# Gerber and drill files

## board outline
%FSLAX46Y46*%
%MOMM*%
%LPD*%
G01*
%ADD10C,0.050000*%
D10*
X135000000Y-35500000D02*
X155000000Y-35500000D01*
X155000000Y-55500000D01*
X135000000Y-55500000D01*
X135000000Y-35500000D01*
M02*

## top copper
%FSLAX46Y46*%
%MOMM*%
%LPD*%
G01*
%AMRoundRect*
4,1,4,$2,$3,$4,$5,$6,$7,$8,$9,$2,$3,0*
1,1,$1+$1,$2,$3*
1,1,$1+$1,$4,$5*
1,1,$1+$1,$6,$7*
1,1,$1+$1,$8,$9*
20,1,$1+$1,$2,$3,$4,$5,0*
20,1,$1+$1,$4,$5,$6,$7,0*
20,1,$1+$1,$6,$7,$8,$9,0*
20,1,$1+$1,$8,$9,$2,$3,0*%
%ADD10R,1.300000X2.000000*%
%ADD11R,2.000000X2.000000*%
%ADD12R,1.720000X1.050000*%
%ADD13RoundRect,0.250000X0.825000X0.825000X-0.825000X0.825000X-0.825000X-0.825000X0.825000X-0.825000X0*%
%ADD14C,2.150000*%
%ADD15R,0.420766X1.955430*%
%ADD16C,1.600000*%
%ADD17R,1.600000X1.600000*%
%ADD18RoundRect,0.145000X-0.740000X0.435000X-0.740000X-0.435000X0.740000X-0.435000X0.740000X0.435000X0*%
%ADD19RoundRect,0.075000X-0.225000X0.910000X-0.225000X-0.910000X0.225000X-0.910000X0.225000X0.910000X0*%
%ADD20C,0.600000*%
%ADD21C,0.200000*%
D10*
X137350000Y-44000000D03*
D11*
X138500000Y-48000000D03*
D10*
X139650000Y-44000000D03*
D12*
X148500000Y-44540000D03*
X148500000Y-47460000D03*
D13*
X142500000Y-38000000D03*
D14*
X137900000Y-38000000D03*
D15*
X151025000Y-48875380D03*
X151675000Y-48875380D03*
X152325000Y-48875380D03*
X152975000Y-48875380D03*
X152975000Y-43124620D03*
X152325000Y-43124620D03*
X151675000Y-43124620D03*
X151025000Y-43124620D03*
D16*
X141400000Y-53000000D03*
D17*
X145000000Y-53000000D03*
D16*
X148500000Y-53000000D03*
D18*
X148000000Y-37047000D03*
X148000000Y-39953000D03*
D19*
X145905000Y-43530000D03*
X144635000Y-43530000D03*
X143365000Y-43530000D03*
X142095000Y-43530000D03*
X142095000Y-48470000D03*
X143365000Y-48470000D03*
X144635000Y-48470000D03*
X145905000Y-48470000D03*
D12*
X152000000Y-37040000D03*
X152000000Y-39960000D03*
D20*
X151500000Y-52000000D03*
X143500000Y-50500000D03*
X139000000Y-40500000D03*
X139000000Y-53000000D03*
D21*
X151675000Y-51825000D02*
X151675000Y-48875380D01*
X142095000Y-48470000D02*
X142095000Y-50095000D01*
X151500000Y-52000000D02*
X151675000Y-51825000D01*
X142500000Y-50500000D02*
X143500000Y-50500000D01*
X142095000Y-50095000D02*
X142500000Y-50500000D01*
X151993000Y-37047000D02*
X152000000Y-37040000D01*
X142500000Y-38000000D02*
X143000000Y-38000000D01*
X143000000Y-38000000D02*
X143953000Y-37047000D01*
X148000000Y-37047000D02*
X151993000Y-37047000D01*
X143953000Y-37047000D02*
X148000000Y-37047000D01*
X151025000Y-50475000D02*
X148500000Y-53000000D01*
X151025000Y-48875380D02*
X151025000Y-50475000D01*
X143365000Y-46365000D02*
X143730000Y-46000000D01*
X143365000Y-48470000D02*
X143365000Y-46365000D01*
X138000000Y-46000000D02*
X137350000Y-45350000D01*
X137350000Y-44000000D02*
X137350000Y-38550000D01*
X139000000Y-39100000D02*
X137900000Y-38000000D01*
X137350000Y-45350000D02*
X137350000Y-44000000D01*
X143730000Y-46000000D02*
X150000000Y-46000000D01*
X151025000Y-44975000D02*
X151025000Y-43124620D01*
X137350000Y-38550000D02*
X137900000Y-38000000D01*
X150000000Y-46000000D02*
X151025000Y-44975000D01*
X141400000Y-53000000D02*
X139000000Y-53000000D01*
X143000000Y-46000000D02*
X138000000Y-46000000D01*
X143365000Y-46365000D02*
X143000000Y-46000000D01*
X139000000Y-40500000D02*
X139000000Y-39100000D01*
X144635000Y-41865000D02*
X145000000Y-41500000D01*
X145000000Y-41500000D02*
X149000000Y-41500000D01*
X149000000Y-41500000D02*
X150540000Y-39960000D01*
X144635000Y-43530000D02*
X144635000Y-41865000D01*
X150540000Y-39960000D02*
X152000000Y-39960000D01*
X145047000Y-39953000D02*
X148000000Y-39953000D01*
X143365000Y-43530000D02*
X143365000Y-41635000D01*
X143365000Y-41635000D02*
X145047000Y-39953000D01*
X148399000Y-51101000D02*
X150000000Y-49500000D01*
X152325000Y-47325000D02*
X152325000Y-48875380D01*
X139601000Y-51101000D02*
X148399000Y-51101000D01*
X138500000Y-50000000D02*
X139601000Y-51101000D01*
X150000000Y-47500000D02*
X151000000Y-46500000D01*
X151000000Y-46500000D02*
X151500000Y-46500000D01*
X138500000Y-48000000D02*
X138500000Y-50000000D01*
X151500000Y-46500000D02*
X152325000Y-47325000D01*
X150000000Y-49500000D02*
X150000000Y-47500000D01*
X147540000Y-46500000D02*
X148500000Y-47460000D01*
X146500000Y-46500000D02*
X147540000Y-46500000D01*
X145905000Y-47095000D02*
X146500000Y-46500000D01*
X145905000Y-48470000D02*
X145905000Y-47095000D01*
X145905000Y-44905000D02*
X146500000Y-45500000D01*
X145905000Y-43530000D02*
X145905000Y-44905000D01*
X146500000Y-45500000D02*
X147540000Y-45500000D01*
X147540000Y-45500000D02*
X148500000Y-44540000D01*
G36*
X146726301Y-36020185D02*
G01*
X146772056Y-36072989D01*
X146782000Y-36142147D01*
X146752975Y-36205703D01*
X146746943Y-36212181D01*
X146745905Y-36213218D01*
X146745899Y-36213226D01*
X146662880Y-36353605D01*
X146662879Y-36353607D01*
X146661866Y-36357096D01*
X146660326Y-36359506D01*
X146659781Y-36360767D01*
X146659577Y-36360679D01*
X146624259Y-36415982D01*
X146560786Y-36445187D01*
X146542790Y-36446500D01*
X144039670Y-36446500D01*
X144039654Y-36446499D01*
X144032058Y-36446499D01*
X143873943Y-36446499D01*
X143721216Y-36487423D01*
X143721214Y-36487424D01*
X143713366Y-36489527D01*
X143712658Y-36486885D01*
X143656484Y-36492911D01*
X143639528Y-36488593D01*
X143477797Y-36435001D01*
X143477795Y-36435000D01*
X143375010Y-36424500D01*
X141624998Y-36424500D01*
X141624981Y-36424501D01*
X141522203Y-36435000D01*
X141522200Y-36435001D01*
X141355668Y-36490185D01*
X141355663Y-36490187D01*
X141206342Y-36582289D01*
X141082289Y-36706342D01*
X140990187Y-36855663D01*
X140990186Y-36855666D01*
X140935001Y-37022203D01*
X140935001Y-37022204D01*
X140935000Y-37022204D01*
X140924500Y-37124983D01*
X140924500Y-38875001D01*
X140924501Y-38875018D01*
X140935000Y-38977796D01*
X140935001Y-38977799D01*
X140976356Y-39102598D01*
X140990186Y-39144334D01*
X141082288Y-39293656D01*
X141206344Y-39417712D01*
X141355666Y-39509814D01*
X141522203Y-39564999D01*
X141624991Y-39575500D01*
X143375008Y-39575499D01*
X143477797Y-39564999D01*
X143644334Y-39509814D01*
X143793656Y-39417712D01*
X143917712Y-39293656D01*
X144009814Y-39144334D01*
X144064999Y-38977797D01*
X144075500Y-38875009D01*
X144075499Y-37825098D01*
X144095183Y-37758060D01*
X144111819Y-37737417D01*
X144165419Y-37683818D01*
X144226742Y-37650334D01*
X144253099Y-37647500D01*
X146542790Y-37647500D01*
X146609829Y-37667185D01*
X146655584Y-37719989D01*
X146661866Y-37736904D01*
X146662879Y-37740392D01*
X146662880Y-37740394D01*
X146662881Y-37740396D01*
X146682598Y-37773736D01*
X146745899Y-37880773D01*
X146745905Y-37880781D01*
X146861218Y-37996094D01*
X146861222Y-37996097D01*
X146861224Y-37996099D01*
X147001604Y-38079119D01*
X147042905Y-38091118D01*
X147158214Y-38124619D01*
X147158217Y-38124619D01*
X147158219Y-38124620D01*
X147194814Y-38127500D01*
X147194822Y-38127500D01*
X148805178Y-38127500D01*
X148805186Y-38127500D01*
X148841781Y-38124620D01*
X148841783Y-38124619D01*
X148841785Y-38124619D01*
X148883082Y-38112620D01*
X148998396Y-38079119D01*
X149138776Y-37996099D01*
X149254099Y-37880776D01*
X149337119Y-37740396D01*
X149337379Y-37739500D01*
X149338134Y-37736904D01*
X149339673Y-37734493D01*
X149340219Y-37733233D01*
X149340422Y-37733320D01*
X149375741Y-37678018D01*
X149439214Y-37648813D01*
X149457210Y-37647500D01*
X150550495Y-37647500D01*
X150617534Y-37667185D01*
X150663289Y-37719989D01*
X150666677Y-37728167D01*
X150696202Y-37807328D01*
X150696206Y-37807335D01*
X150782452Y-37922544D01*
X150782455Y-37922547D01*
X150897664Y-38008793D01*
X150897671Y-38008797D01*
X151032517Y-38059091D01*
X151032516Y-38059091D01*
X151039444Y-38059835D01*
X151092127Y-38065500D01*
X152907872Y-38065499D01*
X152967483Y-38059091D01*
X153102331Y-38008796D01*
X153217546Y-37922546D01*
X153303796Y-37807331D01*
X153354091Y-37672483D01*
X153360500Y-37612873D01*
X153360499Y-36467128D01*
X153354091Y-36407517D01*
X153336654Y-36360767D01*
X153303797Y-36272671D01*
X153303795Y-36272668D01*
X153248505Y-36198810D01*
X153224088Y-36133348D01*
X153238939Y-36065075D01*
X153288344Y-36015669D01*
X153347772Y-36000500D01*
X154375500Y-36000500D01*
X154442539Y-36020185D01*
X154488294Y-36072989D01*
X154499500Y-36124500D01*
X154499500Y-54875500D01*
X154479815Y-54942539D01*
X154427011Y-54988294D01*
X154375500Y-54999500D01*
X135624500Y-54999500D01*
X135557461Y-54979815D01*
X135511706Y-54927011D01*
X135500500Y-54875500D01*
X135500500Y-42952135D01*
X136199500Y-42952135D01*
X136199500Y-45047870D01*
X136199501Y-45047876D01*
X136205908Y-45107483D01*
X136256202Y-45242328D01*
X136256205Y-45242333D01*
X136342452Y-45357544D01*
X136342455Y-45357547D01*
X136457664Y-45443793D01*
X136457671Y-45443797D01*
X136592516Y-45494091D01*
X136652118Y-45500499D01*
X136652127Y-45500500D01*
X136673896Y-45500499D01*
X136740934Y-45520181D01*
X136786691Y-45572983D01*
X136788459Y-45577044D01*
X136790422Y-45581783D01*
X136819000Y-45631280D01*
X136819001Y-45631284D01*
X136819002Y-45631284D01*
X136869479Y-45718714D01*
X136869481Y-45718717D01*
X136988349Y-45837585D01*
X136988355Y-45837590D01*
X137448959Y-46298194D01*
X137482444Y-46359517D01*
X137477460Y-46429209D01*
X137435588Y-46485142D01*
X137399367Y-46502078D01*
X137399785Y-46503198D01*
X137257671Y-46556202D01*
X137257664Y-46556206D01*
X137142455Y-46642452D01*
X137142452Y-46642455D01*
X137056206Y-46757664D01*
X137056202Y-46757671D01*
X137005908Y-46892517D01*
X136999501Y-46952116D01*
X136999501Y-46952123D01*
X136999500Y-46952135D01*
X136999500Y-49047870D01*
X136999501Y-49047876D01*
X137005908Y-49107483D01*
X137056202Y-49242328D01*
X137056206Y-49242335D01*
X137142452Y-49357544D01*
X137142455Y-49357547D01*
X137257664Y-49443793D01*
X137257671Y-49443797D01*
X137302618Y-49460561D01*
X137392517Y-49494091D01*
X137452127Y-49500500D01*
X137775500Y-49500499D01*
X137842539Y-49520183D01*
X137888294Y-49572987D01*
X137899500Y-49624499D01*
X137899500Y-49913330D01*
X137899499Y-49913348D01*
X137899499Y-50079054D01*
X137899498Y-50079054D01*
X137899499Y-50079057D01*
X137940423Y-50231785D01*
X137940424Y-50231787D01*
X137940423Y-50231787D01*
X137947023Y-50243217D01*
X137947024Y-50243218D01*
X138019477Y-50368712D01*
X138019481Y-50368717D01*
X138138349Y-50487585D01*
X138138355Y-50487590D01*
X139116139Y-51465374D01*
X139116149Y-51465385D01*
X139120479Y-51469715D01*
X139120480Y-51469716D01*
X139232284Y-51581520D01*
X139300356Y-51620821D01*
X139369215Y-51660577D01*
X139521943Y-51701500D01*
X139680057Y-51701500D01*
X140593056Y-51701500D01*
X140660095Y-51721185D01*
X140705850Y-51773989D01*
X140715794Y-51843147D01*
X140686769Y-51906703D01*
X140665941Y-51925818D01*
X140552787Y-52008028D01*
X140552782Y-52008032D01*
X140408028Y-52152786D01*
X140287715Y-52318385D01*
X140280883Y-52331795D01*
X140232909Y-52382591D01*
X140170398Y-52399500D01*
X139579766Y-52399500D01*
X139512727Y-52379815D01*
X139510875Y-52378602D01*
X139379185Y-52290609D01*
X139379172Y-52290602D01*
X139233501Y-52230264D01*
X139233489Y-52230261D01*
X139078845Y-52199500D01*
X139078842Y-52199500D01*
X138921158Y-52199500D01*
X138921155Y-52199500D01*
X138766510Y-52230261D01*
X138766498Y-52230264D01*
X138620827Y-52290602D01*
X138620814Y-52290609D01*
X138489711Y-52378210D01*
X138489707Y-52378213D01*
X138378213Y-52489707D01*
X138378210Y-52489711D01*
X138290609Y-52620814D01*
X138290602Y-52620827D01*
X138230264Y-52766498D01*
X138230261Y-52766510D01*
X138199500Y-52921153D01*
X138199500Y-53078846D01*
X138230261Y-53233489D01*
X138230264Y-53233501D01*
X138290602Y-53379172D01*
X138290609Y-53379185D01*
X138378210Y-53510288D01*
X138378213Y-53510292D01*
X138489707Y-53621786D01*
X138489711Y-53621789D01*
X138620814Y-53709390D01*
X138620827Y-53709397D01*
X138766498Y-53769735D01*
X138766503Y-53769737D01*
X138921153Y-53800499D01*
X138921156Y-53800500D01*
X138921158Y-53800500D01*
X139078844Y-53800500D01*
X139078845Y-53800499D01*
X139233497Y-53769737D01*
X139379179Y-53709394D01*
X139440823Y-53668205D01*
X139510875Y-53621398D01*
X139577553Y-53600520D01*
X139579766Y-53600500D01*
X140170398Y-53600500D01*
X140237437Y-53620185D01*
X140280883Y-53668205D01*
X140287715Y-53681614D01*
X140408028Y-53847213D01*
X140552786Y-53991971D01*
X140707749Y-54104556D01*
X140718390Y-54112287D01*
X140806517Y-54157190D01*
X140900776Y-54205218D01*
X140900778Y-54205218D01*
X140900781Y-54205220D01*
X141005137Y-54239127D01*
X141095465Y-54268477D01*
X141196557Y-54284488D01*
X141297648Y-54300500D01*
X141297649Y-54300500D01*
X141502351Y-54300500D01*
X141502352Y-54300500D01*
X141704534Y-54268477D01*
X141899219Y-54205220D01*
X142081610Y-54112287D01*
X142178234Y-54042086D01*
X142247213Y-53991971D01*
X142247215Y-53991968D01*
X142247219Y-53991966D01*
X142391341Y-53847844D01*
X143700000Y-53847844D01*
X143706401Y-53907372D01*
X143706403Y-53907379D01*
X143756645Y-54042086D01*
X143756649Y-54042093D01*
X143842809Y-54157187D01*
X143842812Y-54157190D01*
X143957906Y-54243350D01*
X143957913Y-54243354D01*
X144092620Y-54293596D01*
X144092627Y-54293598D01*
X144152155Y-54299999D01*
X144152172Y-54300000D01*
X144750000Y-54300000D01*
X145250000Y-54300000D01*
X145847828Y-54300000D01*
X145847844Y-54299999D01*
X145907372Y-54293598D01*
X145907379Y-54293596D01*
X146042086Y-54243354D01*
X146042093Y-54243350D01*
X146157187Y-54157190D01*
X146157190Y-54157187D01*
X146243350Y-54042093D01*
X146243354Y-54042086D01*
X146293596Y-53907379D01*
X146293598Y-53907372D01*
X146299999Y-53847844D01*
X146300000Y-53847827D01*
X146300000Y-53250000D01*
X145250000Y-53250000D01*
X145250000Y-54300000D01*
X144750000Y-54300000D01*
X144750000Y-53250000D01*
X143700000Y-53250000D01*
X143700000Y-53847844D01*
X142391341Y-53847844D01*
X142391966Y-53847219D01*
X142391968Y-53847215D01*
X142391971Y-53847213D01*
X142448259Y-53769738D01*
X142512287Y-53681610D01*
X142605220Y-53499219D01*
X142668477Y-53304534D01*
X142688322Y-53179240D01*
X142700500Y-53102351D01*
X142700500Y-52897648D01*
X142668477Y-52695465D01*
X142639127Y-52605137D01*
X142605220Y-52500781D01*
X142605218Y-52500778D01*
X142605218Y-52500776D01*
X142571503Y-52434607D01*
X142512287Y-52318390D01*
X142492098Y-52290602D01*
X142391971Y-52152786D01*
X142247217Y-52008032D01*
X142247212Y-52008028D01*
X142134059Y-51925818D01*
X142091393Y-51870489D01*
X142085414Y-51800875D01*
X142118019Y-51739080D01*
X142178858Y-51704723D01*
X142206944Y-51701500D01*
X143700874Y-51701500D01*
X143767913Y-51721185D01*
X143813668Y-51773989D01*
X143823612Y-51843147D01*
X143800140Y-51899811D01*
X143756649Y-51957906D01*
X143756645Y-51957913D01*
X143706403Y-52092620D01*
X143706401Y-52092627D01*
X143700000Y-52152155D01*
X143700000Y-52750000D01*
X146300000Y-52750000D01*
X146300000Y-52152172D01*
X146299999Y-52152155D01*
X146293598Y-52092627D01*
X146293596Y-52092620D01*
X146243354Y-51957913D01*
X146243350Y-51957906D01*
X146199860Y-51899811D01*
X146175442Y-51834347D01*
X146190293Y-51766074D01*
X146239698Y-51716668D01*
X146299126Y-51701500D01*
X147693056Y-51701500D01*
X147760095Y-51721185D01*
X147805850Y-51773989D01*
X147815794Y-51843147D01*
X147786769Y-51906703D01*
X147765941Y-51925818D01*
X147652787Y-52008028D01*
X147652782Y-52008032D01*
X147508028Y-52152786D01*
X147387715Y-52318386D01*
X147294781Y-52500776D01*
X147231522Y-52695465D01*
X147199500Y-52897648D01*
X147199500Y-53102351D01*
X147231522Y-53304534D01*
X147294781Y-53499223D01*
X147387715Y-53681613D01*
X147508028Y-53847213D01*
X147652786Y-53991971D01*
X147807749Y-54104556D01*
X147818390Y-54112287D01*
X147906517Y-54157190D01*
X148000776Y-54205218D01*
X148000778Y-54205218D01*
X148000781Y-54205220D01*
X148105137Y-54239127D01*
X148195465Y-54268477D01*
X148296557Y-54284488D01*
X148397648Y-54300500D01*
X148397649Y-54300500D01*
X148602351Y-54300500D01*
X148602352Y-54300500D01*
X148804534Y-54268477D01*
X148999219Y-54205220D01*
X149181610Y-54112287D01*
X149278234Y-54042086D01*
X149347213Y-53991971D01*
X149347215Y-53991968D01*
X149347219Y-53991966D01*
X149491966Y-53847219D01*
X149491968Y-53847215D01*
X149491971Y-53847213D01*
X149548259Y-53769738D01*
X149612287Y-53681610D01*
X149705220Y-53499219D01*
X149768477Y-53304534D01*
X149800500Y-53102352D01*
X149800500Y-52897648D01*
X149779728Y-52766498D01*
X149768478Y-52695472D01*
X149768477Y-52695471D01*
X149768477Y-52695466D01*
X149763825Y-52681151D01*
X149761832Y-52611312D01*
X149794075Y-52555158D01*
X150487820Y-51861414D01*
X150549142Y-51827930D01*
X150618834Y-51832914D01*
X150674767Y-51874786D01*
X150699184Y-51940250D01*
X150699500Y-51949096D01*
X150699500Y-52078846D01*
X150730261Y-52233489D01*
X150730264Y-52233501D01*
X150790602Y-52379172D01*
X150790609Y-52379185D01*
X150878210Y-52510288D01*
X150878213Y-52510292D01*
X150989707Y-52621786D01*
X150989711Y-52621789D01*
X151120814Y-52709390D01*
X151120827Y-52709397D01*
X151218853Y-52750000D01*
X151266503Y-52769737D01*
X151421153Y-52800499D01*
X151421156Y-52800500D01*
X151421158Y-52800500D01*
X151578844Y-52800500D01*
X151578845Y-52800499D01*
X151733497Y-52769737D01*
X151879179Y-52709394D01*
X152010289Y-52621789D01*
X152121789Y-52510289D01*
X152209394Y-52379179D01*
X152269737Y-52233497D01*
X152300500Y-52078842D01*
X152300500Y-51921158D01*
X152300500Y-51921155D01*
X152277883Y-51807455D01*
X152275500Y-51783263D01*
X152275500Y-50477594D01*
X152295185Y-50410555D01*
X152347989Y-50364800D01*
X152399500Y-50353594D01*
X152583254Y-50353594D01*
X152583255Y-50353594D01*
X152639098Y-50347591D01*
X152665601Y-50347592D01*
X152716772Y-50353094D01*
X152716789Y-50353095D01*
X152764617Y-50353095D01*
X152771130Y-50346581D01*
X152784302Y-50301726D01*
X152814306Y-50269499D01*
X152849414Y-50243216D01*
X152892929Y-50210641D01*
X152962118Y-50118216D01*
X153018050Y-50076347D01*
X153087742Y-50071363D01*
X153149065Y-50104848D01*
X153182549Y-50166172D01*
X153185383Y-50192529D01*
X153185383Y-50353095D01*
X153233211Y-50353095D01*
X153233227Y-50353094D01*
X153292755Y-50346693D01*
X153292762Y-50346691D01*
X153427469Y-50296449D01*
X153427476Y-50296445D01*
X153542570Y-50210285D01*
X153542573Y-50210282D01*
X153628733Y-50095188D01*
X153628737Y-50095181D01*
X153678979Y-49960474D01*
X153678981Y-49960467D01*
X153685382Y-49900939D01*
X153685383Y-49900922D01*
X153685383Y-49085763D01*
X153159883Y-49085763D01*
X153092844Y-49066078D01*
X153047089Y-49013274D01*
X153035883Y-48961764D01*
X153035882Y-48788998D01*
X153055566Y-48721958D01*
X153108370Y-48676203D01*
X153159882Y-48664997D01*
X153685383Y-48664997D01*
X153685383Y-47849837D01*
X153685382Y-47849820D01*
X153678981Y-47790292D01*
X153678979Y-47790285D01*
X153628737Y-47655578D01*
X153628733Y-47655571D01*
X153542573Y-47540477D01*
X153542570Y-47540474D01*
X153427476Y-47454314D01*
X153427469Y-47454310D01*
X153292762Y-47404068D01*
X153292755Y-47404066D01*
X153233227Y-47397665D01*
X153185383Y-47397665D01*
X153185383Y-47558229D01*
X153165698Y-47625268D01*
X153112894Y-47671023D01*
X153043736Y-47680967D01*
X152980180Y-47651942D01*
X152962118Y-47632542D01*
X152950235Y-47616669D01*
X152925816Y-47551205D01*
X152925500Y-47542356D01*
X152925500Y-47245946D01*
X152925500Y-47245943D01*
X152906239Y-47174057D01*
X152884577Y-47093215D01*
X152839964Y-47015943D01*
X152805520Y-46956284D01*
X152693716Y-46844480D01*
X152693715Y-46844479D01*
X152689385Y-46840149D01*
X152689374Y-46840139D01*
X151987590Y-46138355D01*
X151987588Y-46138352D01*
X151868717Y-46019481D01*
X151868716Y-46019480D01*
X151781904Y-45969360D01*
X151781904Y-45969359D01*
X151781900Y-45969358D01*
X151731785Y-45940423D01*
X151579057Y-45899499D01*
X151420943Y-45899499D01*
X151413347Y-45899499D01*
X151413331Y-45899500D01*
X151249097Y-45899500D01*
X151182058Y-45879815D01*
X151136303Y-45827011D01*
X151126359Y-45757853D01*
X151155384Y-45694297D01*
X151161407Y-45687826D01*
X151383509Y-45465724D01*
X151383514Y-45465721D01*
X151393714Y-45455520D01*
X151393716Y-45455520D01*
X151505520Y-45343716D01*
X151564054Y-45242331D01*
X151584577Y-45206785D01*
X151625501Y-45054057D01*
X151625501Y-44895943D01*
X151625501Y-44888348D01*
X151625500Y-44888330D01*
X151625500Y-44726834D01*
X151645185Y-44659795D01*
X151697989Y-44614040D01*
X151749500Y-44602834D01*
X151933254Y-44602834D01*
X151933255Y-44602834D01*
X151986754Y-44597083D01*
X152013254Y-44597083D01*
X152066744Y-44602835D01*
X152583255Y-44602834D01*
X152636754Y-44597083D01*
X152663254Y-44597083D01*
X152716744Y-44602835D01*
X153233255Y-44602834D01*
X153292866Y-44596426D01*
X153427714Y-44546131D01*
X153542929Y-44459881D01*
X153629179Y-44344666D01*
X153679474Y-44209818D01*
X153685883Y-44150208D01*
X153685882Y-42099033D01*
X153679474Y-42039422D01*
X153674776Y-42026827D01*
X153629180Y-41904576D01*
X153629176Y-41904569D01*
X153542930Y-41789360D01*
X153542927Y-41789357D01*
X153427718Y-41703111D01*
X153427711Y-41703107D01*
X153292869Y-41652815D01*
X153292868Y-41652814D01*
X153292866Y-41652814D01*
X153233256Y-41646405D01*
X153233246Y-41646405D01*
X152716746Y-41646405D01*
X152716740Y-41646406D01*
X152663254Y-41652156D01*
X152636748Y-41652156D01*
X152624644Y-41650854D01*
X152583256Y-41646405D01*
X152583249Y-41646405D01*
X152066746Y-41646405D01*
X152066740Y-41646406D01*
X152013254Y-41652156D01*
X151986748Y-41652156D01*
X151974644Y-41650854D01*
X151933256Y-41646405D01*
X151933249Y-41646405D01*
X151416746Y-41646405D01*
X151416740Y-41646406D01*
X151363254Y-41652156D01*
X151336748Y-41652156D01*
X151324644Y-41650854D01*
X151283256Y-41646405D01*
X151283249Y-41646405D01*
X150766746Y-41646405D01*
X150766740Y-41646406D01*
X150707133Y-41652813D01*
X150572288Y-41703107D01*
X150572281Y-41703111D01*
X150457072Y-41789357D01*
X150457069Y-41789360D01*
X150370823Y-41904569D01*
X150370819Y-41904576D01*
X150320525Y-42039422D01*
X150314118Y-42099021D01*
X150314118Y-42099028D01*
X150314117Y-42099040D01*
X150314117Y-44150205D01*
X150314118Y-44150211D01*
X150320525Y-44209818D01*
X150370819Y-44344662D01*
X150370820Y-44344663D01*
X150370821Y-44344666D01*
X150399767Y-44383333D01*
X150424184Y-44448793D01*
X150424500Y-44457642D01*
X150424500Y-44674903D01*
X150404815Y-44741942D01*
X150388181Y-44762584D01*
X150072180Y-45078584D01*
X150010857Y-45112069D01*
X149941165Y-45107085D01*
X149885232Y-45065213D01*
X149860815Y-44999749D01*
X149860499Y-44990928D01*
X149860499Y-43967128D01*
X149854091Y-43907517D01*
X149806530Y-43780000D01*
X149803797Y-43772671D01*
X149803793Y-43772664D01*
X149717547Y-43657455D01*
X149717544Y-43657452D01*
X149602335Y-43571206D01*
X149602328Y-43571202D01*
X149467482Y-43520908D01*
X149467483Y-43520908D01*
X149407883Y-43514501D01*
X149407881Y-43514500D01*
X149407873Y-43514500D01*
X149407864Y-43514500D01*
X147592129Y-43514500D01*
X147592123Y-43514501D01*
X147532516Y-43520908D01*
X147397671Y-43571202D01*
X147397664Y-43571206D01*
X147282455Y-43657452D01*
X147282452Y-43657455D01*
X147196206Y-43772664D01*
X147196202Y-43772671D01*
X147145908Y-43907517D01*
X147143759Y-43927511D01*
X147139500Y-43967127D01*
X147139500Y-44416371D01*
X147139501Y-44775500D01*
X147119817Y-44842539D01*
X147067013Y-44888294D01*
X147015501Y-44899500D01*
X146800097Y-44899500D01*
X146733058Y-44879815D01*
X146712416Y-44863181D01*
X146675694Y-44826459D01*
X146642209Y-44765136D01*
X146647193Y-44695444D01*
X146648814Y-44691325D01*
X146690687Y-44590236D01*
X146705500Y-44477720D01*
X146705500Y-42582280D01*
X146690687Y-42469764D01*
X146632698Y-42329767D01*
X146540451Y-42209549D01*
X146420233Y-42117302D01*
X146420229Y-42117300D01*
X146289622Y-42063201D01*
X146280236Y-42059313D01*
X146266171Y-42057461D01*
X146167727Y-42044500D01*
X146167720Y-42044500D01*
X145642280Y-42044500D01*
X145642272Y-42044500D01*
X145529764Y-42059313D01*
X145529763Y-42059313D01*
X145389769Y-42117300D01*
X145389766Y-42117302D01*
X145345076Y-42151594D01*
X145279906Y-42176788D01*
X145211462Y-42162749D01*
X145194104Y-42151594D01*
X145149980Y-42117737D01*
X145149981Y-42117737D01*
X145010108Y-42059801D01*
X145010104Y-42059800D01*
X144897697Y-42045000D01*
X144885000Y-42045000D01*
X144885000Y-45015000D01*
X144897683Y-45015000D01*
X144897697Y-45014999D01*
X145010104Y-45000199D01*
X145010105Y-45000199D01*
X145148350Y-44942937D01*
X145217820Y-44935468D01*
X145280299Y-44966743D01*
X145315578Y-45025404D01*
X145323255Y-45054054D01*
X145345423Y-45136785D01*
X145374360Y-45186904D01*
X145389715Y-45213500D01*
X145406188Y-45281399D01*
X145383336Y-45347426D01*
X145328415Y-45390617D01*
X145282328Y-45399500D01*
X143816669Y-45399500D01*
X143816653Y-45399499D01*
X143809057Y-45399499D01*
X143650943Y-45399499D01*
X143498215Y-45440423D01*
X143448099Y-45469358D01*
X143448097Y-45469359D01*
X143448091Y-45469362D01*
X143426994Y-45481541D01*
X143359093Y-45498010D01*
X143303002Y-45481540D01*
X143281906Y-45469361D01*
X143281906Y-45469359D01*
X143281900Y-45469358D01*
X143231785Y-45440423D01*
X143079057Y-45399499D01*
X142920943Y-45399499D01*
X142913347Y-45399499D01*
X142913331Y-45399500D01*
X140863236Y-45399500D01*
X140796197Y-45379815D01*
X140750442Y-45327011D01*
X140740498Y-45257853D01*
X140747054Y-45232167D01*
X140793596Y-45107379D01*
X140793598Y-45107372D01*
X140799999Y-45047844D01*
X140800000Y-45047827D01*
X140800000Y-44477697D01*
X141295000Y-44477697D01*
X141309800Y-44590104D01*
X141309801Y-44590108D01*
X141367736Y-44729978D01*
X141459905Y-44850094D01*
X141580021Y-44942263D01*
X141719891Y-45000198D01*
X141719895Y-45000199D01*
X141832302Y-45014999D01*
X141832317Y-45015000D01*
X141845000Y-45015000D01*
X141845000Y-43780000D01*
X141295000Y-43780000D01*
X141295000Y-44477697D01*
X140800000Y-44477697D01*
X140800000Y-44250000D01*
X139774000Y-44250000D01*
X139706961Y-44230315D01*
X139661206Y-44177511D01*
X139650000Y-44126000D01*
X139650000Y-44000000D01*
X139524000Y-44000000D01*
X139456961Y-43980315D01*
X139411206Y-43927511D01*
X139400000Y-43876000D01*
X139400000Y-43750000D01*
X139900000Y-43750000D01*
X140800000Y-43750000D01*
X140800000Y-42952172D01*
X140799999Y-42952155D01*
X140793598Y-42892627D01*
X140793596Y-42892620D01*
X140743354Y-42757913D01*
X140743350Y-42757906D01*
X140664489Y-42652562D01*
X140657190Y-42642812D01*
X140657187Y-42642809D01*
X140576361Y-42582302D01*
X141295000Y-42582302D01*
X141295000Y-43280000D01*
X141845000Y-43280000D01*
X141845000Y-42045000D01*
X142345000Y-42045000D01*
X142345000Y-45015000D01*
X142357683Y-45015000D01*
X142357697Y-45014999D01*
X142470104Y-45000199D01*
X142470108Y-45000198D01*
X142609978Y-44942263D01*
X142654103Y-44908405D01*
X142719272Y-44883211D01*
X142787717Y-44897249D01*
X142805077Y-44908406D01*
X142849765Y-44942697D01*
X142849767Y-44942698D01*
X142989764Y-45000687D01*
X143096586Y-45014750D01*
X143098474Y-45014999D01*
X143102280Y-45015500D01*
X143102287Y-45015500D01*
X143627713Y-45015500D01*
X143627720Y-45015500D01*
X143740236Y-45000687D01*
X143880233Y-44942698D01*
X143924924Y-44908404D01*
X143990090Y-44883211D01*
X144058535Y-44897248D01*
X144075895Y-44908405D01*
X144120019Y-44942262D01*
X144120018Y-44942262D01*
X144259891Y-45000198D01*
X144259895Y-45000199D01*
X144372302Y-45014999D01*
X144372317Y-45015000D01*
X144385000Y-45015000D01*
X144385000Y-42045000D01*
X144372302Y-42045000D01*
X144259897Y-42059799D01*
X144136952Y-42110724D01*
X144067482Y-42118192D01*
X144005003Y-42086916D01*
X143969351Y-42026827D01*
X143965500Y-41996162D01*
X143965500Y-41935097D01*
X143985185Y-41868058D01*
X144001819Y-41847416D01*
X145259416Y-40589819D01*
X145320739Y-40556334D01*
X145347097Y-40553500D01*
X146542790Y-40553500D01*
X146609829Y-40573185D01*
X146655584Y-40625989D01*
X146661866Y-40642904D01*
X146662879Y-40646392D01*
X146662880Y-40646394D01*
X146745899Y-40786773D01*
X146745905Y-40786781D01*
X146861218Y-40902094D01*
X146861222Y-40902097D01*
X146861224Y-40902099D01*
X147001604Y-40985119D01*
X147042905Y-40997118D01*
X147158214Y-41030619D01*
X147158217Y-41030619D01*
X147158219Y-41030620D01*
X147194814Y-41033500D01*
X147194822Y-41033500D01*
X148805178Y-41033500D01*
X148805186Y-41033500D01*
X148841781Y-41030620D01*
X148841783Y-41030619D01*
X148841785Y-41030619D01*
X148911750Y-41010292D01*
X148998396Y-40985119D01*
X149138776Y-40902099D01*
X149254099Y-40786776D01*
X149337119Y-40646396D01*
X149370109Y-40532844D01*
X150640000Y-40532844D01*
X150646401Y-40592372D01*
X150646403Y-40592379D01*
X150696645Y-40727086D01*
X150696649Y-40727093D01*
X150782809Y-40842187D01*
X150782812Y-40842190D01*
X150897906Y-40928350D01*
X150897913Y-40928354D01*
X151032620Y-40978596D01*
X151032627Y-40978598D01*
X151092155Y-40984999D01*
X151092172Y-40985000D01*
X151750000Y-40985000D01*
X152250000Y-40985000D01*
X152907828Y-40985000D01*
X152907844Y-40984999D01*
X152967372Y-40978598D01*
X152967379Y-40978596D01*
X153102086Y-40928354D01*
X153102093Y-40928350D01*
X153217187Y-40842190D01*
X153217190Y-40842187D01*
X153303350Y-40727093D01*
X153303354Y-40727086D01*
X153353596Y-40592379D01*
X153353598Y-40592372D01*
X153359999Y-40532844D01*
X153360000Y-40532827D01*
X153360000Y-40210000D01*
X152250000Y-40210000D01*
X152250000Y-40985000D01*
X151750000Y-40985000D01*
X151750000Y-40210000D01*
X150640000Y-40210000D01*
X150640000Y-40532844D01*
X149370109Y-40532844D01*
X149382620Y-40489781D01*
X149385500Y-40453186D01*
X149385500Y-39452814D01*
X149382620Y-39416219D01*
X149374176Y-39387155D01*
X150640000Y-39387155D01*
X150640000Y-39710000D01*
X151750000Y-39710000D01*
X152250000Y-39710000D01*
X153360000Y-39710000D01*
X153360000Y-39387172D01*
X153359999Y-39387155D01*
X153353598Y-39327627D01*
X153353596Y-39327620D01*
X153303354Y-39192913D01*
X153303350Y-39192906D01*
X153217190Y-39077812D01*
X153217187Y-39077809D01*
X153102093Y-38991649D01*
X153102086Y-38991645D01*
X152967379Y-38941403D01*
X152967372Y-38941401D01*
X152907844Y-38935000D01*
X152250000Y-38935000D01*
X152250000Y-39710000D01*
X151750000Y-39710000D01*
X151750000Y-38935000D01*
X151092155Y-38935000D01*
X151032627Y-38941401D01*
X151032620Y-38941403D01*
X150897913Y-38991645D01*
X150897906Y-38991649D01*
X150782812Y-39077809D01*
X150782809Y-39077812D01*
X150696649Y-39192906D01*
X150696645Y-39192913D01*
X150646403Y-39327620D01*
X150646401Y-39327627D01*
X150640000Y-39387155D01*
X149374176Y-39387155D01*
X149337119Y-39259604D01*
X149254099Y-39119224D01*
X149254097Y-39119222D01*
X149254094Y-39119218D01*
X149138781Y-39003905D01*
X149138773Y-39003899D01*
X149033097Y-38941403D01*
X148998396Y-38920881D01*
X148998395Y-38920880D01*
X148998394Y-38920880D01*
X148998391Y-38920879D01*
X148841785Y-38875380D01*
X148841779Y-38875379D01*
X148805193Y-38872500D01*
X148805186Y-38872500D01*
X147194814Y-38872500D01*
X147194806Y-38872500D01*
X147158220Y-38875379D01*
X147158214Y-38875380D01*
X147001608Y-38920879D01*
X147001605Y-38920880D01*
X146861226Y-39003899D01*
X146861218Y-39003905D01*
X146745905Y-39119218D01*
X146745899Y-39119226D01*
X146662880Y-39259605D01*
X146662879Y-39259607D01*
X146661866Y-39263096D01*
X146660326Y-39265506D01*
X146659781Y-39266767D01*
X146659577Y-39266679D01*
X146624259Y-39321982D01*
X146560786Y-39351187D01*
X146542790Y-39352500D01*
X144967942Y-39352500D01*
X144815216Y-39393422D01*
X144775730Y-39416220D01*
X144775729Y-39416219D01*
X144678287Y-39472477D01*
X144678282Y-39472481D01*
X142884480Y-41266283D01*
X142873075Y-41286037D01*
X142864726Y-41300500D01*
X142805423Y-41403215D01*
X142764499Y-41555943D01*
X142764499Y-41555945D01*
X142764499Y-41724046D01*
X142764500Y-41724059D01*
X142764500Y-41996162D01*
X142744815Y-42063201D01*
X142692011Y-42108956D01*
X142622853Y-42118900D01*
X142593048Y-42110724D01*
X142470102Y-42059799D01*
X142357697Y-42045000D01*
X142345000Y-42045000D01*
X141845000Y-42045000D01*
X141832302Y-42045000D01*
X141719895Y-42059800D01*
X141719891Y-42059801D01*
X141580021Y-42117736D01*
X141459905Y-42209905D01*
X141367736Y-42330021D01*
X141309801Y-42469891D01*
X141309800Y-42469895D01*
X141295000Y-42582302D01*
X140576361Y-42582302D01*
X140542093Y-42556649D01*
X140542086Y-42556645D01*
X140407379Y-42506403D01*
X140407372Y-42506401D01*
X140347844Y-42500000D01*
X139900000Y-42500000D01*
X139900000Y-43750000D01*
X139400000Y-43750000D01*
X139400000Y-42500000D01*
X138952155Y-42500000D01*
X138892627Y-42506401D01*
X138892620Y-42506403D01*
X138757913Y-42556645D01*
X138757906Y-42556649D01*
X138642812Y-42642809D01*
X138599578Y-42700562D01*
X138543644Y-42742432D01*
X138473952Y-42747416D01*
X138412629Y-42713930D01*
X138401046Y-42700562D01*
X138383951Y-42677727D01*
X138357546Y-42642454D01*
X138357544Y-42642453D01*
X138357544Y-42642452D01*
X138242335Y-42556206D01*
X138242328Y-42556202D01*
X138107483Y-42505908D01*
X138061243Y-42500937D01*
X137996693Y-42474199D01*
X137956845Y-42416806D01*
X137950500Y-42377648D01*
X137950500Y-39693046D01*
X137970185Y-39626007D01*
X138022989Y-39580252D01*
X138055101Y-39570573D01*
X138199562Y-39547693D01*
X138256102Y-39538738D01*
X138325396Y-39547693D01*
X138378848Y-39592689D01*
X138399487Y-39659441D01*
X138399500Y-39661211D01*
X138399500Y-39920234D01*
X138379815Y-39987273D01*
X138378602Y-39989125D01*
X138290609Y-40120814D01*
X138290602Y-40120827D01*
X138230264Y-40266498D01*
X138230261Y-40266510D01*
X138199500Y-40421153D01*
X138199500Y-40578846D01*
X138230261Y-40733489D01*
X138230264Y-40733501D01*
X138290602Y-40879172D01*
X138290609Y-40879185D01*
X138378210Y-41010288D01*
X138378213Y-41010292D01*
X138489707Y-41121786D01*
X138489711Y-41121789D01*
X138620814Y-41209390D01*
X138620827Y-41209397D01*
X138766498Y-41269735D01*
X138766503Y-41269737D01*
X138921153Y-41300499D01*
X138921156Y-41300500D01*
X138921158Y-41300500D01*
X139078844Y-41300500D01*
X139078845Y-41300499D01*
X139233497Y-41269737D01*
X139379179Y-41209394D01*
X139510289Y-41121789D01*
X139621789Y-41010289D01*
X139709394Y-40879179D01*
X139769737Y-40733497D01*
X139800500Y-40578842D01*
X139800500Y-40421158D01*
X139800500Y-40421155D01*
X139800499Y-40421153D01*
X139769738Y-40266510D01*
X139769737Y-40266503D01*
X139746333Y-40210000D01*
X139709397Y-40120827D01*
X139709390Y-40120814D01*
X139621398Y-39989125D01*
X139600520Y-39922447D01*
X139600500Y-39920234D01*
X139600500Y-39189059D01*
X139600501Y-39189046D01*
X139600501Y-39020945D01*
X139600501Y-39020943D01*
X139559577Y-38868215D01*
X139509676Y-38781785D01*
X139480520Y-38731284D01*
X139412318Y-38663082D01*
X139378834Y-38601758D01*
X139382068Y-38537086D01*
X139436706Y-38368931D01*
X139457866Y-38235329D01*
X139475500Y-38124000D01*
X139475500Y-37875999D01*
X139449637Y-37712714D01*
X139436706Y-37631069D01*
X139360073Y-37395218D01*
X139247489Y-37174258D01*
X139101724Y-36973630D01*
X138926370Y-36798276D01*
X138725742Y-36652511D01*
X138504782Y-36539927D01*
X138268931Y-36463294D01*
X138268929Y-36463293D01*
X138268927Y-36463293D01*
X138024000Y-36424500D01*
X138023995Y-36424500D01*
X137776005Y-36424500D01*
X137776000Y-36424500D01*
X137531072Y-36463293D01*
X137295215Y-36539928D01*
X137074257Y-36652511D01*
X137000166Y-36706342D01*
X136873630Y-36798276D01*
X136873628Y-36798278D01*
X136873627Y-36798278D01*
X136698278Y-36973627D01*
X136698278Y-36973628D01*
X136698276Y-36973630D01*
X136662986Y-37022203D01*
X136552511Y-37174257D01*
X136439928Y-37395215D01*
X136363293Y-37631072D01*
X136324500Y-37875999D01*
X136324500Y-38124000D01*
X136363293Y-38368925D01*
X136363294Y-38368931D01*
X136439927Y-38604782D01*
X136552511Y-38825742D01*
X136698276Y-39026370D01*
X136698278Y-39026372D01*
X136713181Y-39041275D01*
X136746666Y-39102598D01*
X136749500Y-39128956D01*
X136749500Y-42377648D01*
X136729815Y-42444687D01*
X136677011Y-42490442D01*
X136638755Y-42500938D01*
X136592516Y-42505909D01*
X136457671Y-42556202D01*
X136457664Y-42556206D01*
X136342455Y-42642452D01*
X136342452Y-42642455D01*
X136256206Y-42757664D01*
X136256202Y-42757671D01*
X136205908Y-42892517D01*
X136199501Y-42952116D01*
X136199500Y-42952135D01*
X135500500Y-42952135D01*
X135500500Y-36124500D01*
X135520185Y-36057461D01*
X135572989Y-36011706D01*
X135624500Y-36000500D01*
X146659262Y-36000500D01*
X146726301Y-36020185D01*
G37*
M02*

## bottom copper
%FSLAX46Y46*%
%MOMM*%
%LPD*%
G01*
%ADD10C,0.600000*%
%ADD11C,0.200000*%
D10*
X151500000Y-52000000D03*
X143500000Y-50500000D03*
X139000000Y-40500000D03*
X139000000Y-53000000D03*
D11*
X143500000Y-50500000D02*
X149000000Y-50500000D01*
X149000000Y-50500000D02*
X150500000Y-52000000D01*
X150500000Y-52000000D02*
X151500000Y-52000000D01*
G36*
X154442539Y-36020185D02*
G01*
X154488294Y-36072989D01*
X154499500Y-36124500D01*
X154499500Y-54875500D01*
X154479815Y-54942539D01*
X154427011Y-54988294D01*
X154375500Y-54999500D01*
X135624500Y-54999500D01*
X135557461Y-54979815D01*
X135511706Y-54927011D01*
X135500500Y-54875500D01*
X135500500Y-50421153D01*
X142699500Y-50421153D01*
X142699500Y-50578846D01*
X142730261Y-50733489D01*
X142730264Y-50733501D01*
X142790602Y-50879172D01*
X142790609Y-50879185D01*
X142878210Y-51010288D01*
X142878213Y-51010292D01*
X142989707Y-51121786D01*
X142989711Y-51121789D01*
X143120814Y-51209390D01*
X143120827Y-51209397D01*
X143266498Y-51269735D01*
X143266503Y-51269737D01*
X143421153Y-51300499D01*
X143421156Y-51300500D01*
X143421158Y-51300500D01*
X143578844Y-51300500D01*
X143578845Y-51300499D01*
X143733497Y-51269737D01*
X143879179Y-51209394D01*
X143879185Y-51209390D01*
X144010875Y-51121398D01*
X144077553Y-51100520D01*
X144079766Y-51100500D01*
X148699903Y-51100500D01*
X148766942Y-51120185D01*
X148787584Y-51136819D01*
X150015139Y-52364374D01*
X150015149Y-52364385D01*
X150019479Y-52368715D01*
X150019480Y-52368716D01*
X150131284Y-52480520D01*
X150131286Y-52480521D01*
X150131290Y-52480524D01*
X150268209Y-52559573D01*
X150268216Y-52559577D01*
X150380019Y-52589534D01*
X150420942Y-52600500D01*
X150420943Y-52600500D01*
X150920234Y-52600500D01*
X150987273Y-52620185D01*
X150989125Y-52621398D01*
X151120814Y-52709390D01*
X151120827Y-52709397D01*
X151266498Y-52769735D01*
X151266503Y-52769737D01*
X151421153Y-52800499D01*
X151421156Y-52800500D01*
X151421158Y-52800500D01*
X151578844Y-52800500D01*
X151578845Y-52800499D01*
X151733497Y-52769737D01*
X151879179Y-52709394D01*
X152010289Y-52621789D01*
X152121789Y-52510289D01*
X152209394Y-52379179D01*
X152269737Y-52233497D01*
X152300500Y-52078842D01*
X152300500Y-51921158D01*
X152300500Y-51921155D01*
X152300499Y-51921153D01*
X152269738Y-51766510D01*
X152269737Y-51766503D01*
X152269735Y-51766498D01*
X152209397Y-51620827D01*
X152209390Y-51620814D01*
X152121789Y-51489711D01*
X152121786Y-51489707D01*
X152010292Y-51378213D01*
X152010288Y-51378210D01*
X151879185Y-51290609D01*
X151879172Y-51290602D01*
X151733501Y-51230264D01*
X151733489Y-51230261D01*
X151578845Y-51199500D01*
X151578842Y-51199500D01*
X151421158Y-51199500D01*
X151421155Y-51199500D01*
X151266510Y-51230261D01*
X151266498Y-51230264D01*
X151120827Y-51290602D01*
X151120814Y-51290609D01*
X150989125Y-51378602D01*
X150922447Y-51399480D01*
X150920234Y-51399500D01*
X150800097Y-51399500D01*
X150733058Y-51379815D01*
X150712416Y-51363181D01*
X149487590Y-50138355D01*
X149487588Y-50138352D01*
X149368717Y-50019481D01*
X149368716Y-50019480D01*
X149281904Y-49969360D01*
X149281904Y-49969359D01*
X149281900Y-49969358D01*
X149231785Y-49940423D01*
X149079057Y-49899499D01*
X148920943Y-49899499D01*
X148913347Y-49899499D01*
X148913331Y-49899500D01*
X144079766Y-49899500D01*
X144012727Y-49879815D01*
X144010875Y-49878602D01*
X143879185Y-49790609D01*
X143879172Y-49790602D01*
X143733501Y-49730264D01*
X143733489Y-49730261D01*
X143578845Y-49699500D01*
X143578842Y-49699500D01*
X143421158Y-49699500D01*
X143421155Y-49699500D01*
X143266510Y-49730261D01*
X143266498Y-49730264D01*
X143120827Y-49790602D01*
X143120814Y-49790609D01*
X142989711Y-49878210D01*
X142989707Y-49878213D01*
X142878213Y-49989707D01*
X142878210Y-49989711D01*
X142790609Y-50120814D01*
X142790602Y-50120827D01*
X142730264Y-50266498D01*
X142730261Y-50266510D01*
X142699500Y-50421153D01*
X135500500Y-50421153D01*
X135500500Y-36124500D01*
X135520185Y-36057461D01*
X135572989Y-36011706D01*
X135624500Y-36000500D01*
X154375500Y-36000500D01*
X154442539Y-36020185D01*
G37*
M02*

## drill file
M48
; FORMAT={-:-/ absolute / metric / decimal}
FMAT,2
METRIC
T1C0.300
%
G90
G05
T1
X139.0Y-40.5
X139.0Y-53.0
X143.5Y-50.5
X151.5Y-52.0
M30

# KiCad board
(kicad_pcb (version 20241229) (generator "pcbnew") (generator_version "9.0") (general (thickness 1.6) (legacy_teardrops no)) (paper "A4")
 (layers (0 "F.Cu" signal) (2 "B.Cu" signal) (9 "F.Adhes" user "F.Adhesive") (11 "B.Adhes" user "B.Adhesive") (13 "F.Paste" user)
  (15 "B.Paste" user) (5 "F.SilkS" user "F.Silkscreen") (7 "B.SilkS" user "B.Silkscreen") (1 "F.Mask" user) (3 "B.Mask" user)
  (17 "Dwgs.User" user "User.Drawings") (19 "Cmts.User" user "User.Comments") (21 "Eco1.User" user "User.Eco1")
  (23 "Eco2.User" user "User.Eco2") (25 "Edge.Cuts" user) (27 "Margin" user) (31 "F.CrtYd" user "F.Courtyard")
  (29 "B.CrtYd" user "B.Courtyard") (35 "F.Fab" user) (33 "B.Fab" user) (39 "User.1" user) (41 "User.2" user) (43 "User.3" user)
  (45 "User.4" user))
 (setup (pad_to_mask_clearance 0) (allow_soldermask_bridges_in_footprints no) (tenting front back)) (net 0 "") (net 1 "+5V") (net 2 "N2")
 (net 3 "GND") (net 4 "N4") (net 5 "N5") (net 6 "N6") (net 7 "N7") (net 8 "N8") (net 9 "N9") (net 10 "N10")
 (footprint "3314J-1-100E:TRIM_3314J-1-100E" (layer "F.Cu") (at 138.5 46 180)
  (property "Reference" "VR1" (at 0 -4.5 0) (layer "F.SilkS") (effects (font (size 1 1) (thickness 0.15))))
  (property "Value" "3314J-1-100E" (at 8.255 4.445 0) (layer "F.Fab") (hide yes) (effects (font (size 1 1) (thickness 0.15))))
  (pad "1" smd rect (at 1.15 2 180) (size 1.3 2) (layers "F.Cu" "F.Mask" "F.Paste") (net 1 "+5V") (solder_mask_margin 0.102))
  (pad "2" smd rect (at 0 -2 180) (size 2 2) (layers "F.Cu" "F.Mask" "F.Paste") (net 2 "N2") (solder_mask_margin 0.102))
  (pad "3" smd rect (at -1.15 2 180) (size 1.3 2) (layers "F.Cu" "F.Mask" "F.Paste") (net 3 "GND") (solder_mask_margin 0.102)))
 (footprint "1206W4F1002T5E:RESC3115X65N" (layer "F.Cu") (at 148.5 46 -90)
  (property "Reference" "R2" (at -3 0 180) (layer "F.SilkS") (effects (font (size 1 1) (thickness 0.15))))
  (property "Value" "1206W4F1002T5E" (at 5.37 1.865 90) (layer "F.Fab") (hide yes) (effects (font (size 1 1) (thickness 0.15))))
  (pad "1" smd rect (at -1.46 0 270) (size 1.05 1.72) (layers "F.Cu" "F.Mask" "F.Paste") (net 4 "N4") (solder_mask_margin 0.102))
  (pad "2" smd rect (at 1.46 0 270) (size 1.05 1.72) (layers "F.Cu" "F.Mask" "F.Paste") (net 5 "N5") (solder_mask_margin 0.102)))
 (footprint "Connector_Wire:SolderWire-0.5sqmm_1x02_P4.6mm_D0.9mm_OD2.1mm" (layer "F.Cu") (at 142.5 38 180)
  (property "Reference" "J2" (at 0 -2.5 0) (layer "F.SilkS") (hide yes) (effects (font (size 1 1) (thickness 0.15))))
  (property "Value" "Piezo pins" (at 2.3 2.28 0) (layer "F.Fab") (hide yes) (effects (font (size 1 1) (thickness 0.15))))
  (pad "1" smd roundrect (at 0 0 180) (size 2.15 2.15) (layers "F.Cu" "F.Mask" "F.Paste") (roundrect_rratio 0.116279) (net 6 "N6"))
  (pad "2" smd circle (at 4.6 0 180) (size 2.15 2.15) (layers "F.Cu" "F.Mask" "F.Paste") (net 1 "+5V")))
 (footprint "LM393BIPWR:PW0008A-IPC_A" (layer "F.Cu") (at 152 46 90)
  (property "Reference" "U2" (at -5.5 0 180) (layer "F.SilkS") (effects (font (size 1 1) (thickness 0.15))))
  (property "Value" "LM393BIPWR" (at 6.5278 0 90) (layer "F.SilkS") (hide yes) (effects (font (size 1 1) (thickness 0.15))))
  (pad "1" smd rect (at -2.87538 -0.975 90) (size 1.95543 0.420766) (layers "F.Cu" "F.Mask" "F.Paste") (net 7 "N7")
   (solder_mask_margin 0.102))
  (pad "2" smd rect (at -2.87538 -0.325 90) (size 1.95543 0.420766) (layers "F.Cu" "F.Mask" "F.Paste") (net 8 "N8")
   (solder_mask_margin 0.102))
  (pad "3" smd rect (at -2.87538 0.325 90) (size 1.95543 0.420766) (layers "F.Cu" "F.Mask" "F.Paste") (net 2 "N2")
   (solder_mask_margin 0.102))
  (pad "4" smd rect (at -2.87538 0.975 90) (size 1.95543 0.420766) (layers "F.Cu" "F.Mask" "F.Paste") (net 3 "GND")
   (solder_mask_margin 0.102))
  (pad "5" smd rect (at 2.87538 0.975 90) (size 1.95543 0.420766) (layers "F.Cu" "F.Mask" "F.Paste") (solder_mask_margin 0.102))
  (pad "6" smd rect (at 2.87538 0.325 90) (size 1.95543 0.420766) (layers "F.Cu" "F.Mask" "F.Paste") (solder_mask_margin 0.102))
  (pad "7" smd rect (at 2.87538 -0.325 90) (size 1.95543 0.420766) (layers "F.Cu" "F.Mask" "F.Paste") (solder_mask_margin 0.102))
  (pad "8" smd rect (at 2.87538 -0.975 90) (size 1.95543 0.420766) (layers "F.Cu" "F.Mask" "F.Paste") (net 1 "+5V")
   (solder_mask_margin 0.102)))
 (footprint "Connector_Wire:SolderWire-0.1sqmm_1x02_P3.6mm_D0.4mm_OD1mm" (layer "F.Cu") (at 141.4 53)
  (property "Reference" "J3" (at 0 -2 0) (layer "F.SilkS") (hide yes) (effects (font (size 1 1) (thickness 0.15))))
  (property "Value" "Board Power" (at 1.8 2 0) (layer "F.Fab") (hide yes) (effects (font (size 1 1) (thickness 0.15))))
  (pad "1" smd circle (at 0 0) (size 1.6 1.6) (layers "F.Cu" "F.Mask" "F.Paste") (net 1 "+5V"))
  (pad "2" smd rect (at 3.6 0) (size 1.6 1.6) (layers "F.Cu" "F.Mask" "F.Paste") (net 3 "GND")))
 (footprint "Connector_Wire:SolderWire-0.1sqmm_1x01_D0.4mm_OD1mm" (layer "F.Cu") (at 148.5 53)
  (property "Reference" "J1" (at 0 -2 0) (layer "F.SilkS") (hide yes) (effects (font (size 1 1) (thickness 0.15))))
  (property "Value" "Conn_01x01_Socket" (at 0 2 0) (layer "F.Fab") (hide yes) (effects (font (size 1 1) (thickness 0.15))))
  (pad "1" smd circle (at 0 0) (size 1.6 1.6) (layers "F.Cu" "F.Mask" "F.Paste") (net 7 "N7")))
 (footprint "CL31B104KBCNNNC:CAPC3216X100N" (layer "F.Cu") (at 148 38.5 -90)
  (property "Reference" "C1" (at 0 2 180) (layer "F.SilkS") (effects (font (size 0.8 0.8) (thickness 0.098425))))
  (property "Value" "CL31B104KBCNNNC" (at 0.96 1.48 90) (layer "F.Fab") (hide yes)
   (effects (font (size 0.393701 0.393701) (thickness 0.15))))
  (pad "1" smd roundrect (at -1.453 0 270) (size 1.16 1.77) (layers "F.Cu" "F.Mask" "F.Paste") (roundrect_rratio 0.125) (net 6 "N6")
   (solder_mask_margin 0.102))
  (pad "2" smd roundrect (at 1.453 0 270) (size 1.16 1.77) (layers "F.Cu" "F.Mask" "F.Paste") (roundrect_rratio 0.125) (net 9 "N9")
   (solder_mask_margin 0.102)))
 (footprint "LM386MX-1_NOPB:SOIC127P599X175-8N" (layer "F.Cu") (at 144 46 -90)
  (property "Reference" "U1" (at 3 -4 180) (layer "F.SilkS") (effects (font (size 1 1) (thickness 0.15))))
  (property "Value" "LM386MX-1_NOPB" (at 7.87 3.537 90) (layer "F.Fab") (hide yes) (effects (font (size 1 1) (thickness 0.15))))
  (pad "1" smd roundrect (at -2.47 -1.905 270) (size 1.97 0.6) (layers "F.Cu" "F.Mask" "F.Paste") (roundrect_rratio 0.125) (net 4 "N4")
   (solder_mask_margin 0.102))
  (pad "2" smd roundrect (at -2.47 -0.635 270) (size 1.97 0.6) (layers "F.Cu" "F.Mask" "F.Paste") (roundrect_rratio 0.125) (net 3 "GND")
   (solder_mask_margin 0.102))
  (pad "3" smd roundrect (at -2.47 0.635 270) (size 1.97 0.6) (layers "F.Cu" "F.Mask" "F.Paste") (roundrect_rratio 0.125) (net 9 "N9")
   (solder_mask_margin 0.102))
  (pad "4" smd roundrect (at -2.47 1.905 270) (size 1.97 0.6) (layers "F.Cu" "F.Mask" "F.Paste") (roundrect_rratio 0.125) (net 3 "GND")
   (solder_mask_margin 0.102))
  (pad "5" smd roundrect (at 2.47 1.905 270) (size 1.97 0.6) (layers "F.Cu" "F.Mask" "F.Paste") (roundrect_rratio 0.125) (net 8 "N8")
   (solder_mask_margin 0.102))
  (pad "6" smd roundrect (at 2.47 0.635 270) (size 1.97 0.6) (layers "F.Cu" "F.Mask" "F.Paste") (roundrect_rratio 0.125) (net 1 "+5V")
   (solder_mask_margin 0.102))
  (pad "7" smd roundrect (at 2.47 -0.635 270) (size 1.97 0.6) (layers "F.Cu" "F.Mask" "F.Paste") (roundrect_rratio 0.125) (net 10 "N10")
   (solder_mask_margin 0.102))
  (pad "8" smd roundrect (at 2.47 -1.905 270) (size 1.97 0.6) (layers "F.Cu" "F.Mask" "F.Paste") (roundrect_rratio 0.125) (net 5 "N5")
   (solder_mask_margin 0.102)))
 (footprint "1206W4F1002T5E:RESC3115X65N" (layer "F.Cu") (at 152 38.5 -90)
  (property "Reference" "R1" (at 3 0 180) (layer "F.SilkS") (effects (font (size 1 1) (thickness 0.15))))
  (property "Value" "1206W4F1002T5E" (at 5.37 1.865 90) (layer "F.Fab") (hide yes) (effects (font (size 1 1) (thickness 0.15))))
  (pad "1" smd rect (at -1.46 0 270) (size 1.05 1.72) (layers "F.Cu" "F.Mask" "F.Paste") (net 6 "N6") (solder_mask_margin 0.102))
  (pad "2" smd rect (at 1.46 0 270) (size 1.05 1.72) (layers "F.Cu" "F.Mask" "F.Paste") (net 3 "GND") (solder_mask_margin 0.102)))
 (gr_rect (start 135 35.5) (end 155 55.5) (stroke (width 0.05) (type default)) (fill no) (layer "Edge.Cuts"))
 (segment (start 151.675 51.825) (end 151.675 48.87538) (width 0.2) (layer "F.Cu") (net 8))
 (segment (start 142.095 48.47) (end 142.095 50.095) (width 0.2) (layer "F.Cu") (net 8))
 (segment (start 151.5 52) (end 151.675 51.825) (width 0.2) (layer "F.Cu") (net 8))
 (segment (start 142.5 50.5) (end 143.5 50.5) (width 0.2) (layer "F.Cu") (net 8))
 (segment (start 142.095 50.095) (end 142.5 50.5) (width 0.2) (layer "F.Cu") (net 8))
 (via (at 151.5 52) (size 0.6) (drill 0.3) (layers "F.Cu" "B.Cu") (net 8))
 (via (at 143.5 50.5) (size 0.6) (drill 0.3) (layers "F.Cu" "B.Cu") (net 8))
 (segment (start 143.5 50.5) (end 149 50.5) (width 0.2) (layer "B.Cu") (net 8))
 (segment (start 149 50.5) (end 150.5 52) (width 0.2) (layer "B.Cu") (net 8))
 (segment (start 150.5 52) (end 151.5 52) (width 0.2) (layer "B.Cu") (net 8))
 (segment (start 151.993 37.047) (end 152 37.04) (width 0.2) (layer "F.Cu") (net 6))
 (segment (start 142.5 38) (end 143 38) (width 0.2) (layer "F.Cu") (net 6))
 (segment (start 143 38) (end 143.953 37.047) (width 0.2) (layer "F.Cu") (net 6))
 (segment (start 148 37.047) (end 151.993 37.047) (width 0.2) (layer "F.Cu") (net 6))
 (segment (start 143.953 37.047) (end 148 37.047) (width 0.2) (layer "F.Cu") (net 6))
 (segment (start 151.025 50.475) (end 148.5 53) (width 0.2) (layer "F.Cu") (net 7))
 (segment (start 151.025 48.87538) (end 151.025 50.475) (width 0.2) (layer "F.Cu") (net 7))
 (segment (start 143.365 46.365) (end 143.73 46) (width 0.2) (layer "F.Cu") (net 1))
 (segment (start 143.365 48.47) (end 143.365 46.365) (width 0.2) (layer "F.Cu") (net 1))
 (segment (start 138 46) (end 137.35 45.35) (width 0.2) (layer "F.Cu") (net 1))
 (segment (start 137.35 44) (end 137.35 38.55) (width 0.2) (layer "F.Cu") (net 1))
 (segment (start 139 39.1) (end 137.9 38) (width 0.2) (layer "F.Cu") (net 1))
 (segment (start 137.35 45.35) (end 137.35 44) (width 0.2) (layer "F.Cu") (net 1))
 (segment (start 143.73 46) (end 150 46) (width 0.2) (layer "F.Cu") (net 1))
 (segment (start 151.025 44.975) (end 151.025 43.12462) (width 0.2) (layer "F.Cu") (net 1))
 (segment (start 137.35 38.55) (end 137.9 38) (width 0.2) (layer "F.Cu") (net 1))
 (segment (start 150 46) (end 151.025 44.975) (width 0.2) (layer "F.Cu") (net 1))
 (segment (start 141.4 53) (end 139 53) (width 0.2) (layer "F.Cu") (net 1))
 (segment (start 143 46) (end 138 46) (width 0.2) (layer "F.Cu") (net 1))
 (segment (start 143.365 46.365) (end 143 46) (width 0.2) (layer "F.Cu") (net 1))
 (segment (start 139 40.5) (end 139 39.1) (width 0.2) (layer "F.Cu") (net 1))
 (via (at 139 40.5) (size 0.6) (drill 0.3) (layers "F.Cu" "B.Cu") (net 1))
 (via (at 139 53) (size 0.6) (drill 0.3) (layers "F.Cu" "B.Cu") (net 1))
 (segment (start 144.635 41.865) (end 145 41.5) (width 0.2) (layer "F.Cu") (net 3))
 (segment (start 145 41.5) (end 149 41.5) (width 0.2) (layer "F.Cu") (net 3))
 (segment (start 149 41.5) (end 150.54 39.96) (width 0.2) (layer "F.Cu") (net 3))
 (segment (start 144.635 43.53) (end 144.635 41.865) (width 0.2) (layer "F.Cu") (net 3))
 (segment (start 150.54 39.96) (end 152 39.96) (width 0.2) (layer "F.Cu") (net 3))
 (segment (start 145.047 39.953) (end 148 39.953) (width 0.2) (layer "F.Cu") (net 9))
 (segment (start 143.365 43.53) (end 143.365 41.635) (width 0.2) (layer "F.Cu") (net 9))
 (segment (start 143.365 41.635) (end 145.047 39.953) (width 0.2) (layer "F.Cu") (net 9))
 (segment (start 148.399 51.101) (end 150 49.5) (width 0.2) (layer "F.Cu") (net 2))
 (segment (start 152.325 47.325) (end 152.325 48.87538) (width 0.2) (layer "F.Cu") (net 2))
 (segment (start 139.601 51.101) (end 148.399 51.101) (width 0.2) (layer "F.Cu") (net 2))
 (segment (start 138.5 50) (end 139.601 51.101) (width 0.2) (layer "F.Cu") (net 2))
 (segment (start 150 47.5) (end 151 46.5) (width 0.2) (layer "F.Cu") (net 2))
 (segment (start 151 46.5) (end 151.5 46.5) (width 0.2) (layer "F.Cu") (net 2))
 (segment (start 138.5 48) (end 138.5 50) (width 0.2) (layer "F.Cu") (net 2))
 (segment (start 151.5 46.5) (end 152.325 47.325) (width 0.2) (layer "F.Cu") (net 2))
 (segment (start 150 49.5) (end 150 47.5) (width 0.2) (layer "F.Cu") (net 2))
 (segment (start 147.54 46.5) (end 148.5 47.46) (width 0.2) (layer "F.Cu") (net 5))
 (segment (start 146.5 46.5) (end 147.54 46.5) (width 0.2) (layer "F.Cu") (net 5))
 (segment (start 145.905 47.095) (end 146.5 46.5) (width 0.2) (layer "F.Cu") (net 5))
 (segment (start 145.905 48.47) (end 145.905 47.095) (width 0.2) (layer "F.Cu") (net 5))
 (segment (start 145.905 44.905) (end 146.5 45.5) (width 0.2) (layer "F.Cu") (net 4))
 (segment (start 145.905 43.53) (end 145.905 44.905) (width 0.2) (layer "F.Cu") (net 4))
 (segment (start 146.5 45.5) (end 147.54 45.5) (width 0.2) (layer "F.Cu") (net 4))
 (segment (start 147.54 45.5) (end 148.5 44.54) (width 0.2) (layer "F.Cu") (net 4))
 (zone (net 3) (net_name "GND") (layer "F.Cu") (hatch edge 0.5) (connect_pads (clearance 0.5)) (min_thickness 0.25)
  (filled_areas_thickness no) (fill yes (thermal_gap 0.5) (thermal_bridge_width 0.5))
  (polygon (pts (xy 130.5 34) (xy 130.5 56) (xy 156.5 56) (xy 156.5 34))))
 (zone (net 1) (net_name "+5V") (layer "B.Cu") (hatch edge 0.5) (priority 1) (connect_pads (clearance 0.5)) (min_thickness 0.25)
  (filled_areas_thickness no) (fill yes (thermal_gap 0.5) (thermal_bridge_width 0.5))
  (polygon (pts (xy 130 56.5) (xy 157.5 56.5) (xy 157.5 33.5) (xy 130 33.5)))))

